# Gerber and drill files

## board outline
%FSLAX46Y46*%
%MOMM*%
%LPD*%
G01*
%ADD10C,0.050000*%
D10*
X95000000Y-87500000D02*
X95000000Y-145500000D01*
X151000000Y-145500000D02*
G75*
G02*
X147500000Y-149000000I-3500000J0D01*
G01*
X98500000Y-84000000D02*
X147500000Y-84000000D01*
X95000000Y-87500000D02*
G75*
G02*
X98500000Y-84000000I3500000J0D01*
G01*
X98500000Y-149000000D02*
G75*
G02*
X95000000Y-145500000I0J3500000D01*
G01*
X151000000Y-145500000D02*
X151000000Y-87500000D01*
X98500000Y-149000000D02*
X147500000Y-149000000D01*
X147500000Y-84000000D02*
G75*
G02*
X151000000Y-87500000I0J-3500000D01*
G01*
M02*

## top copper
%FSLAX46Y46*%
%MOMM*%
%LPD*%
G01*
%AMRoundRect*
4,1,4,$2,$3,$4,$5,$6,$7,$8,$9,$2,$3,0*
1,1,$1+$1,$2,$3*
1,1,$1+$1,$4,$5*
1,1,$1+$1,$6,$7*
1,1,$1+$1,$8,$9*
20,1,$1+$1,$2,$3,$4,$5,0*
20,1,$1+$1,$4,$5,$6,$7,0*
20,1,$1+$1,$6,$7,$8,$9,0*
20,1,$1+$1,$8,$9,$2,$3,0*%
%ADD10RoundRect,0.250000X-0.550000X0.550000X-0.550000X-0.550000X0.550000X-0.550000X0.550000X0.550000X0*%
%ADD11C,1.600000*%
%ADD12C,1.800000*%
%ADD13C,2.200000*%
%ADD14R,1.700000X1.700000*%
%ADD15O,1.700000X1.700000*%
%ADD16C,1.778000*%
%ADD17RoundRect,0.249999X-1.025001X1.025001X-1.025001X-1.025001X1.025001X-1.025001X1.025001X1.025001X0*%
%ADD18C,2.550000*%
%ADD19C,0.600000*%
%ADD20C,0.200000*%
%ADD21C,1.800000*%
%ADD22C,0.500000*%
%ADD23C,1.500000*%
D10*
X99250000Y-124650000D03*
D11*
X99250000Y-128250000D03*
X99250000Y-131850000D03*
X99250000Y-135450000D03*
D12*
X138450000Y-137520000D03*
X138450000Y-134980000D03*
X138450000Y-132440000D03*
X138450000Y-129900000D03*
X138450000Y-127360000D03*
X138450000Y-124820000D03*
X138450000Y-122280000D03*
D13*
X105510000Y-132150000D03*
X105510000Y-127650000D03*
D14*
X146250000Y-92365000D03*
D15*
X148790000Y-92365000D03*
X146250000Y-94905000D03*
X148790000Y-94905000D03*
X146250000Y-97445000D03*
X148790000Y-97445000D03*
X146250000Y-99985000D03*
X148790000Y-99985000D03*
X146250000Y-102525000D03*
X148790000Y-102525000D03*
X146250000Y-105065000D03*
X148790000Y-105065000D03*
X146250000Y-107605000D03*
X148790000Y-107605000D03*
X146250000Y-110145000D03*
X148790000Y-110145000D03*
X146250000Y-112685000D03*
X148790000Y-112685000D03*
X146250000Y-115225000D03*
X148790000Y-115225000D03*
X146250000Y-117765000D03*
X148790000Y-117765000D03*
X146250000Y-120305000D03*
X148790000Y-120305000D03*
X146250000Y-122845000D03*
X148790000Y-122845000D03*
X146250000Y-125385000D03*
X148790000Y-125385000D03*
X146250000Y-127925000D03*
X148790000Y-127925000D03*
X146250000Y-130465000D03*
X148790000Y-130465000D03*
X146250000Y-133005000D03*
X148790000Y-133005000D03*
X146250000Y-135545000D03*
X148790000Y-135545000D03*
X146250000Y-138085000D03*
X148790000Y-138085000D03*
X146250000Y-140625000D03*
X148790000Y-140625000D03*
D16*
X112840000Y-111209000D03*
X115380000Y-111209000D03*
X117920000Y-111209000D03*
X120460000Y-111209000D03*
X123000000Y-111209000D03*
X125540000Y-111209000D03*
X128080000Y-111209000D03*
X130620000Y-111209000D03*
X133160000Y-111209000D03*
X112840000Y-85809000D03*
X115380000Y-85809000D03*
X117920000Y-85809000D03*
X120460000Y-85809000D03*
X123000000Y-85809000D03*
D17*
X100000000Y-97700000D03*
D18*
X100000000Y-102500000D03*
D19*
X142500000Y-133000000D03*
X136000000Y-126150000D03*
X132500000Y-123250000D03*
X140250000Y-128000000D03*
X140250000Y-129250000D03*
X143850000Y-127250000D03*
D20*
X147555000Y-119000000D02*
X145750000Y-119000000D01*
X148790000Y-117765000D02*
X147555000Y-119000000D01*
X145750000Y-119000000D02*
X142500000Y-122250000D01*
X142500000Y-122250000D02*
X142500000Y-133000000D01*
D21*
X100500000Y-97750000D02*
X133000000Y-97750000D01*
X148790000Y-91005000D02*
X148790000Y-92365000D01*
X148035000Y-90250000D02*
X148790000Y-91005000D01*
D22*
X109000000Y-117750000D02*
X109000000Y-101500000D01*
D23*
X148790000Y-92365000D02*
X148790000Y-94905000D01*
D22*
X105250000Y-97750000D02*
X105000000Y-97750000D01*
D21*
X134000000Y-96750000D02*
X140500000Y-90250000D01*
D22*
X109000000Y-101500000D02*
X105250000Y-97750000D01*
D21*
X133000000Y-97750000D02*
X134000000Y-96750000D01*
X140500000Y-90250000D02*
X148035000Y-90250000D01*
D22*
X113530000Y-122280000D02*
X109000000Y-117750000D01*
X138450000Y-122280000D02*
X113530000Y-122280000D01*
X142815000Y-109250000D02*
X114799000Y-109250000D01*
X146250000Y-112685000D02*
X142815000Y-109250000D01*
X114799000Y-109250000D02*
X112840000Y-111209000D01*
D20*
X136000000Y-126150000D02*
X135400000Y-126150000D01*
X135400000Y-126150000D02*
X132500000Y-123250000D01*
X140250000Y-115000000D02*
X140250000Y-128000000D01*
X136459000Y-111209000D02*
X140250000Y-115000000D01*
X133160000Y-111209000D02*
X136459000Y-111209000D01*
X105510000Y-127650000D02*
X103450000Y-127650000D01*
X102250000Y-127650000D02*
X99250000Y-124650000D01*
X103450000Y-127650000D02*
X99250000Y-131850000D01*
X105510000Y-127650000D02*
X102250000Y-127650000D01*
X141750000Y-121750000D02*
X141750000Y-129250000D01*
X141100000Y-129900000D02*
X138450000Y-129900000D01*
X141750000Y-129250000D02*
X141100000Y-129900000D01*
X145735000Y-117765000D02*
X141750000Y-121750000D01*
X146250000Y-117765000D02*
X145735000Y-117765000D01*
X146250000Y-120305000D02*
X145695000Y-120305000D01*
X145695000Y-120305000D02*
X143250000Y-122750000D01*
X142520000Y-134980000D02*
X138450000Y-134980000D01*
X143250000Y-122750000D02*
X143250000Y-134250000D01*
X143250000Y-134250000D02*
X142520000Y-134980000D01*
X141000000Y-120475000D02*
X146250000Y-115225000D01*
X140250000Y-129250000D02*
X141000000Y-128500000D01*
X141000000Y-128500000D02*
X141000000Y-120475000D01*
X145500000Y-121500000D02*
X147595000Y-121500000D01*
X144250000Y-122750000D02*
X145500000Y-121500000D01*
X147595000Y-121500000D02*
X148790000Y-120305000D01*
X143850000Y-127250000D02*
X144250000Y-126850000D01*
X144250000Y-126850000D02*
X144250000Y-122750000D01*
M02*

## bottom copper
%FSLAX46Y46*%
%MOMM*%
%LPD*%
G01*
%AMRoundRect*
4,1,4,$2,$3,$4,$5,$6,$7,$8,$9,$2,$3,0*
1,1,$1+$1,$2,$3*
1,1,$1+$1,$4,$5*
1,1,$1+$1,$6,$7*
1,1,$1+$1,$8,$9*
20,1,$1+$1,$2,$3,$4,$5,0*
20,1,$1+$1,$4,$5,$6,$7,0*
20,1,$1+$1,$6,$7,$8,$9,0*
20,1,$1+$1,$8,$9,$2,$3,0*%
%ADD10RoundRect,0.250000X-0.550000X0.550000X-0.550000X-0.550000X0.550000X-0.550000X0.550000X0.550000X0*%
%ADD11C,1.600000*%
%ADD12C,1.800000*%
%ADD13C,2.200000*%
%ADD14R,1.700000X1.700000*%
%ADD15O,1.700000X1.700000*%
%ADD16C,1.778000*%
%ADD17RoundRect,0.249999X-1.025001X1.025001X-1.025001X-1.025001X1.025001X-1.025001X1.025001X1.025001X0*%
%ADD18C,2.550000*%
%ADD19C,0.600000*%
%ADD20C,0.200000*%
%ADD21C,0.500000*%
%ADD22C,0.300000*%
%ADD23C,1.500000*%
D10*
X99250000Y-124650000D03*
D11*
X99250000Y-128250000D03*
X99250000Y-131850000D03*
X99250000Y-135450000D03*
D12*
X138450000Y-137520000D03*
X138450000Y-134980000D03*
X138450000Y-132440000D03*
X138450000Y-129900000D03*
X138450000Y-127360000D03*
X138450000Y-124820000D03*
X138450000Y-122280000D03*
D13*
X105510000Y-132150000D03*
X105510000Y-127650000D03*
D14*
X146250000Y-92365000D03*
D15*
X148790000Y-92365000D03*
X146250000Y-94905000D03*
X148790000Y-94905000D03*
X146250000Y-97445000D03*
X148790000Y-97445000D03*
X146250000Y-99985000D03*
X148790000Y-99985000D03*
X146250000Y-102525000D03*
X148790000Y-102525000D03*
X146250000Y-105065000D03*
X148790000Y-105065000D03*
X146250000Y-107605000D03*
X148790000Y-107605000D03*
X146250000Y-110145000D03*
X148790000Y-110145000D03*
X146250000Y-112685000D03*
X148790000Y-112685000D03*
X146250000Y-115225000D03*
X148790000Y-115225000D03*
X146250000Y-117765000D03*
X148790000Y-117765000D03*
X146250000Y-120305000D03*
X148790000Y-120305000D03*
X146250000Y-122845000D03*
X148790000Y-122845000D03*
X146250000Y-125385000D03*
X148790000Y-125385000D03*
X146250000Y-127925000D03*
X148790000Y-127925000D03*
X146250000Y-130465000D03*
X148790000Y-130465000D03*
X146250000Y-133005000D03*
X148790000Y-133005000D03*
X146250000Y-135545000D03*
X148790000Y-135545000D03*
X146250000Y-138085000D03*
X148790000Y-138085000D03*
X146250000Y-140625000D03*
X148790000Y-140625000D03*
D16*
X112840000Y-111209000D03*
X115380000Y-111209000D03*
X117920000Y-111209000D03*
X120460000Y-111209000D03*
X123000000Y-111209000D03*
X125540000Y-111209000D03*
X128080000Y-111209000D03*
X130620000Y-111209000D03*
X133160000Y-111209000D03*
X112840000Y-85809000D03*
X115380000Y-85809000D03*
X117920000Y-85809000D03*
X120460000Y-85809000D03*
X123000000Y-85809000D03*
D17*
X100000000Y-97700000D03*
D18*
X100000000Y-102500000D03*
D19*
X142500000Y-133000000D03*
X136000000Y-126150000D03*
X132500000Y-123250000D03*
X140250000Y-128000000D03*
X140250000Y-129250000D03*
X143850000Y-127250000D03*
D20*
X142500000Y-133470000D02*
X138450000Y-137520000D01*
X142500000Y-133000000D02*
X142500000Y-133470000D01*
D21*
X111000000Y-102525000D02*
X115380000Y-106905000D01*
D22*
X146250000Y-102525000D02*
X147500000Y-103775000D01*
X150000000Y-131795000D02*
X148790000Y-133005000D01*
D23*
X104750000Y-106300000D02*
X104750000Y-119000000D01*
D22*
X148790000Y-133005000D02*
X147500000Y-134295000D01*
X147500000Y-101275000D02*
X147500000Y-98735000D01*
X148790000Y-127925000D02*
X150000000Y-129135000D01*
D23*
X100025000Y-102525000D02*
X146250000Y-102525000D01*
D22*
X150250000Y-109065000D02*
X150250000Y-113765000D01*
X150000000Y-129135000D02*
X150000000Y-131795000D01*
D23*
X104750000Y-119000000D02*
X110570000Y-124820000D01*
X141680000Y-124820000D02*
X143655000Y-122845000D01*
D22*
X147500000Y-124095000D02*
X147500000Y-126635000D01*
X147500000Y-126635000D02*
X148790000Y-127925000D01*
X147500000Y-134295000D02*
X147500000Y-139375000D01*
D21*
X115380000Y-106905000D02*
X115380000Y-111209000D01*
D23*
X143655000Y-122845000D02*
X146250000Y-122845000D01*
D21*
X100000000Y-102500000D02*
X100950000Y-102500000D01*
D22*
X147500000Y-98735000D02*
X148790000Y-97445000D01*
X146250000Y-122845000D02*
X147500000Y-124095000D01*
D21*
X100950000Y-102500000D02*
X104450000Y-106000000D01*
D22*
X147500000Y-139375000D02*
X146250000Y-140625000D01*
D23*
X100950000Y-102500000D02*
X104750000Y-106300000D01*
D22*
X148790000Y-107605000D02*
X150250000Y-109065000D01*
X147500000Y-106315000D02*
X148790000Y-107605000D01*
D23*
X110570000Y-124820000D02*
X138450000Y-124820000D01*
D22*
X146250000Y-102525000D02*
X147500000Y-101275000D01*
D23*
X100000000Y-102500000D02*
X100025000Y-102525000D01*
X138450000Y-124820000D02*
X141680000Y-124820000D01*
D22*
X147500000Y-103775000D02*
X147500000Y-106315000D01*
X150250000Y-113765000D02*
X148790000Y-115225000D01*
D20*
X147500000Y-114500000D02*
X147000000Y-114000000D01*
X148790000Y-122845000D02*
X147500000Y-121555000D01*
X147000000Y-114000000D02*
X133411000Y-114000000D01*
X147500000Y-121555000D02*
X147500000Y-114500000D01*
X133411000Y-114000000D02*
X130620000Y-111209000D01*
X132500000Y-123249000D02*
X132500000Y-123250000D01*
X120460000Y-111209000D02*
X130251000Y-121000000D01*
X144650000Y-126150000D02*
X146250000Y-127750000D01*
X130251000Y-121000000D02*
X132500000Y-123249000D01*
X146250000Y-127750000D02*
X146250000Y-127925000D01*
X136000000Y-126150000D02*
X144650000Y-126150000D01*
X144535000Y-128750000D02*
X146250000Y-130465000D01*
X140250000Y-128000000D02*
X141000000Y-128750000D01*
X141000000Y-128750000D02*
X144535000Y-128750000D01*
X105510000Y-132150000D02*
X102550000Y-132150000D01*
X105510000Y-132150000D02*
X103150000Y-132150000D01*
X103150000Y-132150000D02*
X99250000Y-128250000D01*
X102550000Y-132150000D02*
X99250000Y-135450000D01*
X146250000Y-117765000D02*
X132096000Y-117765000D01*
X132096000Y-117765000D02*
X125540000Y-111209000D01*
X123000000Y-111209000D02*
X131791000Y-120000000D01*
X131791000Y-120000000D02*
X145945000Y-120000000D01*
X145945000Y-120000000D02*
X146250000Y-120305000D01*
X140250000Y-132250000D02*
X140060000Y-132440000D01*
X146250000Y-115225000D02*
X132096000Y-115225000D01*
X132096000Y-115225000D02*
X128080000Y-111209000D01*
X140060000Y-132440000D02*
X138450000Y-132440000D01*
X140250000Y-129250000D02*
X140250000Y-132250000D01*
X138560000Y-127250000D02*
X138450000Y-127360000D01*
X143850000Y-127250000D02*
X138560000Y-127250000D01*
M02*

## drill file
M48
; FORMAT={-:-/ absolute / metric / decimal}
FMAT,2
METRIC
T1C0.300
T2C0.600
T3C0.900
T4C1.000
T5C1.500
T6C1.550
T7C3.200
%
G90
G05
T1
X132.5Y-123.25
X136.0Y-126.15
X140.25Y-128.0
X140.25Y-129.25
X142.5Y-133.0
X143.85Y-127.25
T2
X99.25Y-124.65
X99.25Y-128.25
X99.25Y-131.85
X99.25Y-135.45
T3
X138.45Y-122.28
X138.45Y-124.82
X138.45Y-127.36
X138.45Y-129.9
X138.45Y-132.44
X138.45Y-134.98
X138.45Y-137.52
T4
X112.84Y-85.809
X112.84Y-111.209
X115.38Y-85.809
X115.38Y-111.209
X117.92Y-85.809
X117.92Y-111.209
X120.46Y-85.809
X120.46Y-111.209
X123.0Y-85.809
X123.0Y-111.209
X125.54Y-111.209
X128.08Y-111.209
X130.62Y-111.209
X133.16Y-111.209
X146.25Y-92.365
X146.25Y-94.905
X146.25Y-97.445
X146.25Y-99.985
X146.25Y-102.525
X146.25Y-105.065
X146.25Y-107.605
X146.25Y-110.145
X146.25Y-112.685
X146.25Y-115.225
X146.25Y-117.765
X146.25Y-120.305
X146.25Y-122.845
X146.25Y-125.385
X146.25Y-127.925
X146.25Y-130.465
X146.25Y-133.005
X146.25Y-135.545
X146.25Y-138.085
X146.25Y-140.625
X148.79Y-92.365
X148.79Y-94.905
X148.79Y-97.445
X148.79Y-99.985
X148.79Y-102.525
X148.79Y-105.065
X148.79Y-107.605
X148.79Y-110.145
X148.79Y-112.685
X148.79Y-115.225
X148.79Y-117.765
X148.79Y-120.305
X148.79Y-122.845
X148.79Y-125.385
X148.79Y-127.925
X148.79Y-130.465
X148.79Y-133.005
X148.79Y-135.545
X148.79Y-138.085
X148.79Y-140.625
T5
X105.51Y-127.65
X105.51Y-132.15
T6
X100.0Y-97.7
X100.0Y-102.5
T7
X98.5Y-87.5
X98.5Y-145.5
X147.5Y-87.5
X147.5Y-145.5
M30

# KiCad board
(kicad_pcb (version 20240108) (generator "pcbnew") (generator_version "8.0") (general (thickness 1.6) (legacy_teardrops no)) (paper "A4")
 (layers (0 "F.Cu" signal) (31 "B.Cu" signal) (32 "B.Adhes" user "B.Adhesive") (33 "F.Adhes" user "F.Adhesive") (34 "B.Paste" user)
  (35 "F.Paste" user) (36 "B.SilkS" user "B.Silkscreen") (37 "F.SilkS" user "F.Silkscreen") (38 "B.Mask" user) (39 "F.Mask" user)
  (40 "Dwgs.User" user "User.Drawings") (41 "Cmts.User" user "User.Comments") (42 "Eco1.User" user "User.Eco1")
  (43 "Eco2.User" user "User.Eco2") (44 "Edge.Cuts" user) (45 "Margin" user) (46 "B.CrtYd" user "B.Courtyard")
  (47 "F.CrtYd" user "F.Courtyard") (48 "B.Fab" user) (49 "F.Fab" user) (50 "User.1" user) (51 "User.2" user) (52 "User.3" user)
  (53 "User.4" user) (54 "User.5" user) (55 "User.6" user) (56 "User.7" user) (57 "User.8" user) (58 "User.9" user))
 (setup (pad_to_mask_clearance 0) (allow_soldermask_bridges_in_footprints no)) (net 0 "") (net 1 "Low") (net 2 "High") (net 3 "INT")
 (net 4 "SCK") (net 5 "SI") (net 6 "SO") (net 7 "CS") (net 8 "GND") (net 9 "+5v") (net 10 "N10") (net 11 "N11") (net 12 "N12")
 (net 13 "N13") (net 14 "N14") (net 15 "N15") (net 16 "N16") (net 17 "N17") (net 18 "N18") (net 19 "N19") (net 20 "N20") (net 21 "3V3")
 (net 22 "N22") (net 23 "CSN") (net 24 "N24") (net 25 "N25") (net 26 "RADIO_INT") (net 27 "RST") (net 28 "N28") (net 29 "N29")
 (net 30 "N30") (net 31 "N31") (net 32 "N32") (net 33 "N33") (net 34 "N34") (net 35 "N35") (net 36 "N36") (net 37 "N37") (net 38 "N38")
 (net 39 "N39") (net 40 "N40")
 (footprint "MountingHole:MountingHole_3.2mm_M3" (layer "F.Cu") (at 147.5 87.5 180)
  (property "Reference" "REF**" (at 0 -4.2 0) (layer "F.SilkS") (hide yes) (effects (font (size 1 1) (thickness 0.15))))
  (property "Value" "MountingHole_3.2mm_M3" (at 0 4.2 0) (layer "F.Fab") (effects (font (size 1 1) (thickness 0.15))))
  (pad "" np_thru_hole circle (at 0 0 180) (size 3.2 3.2) (drill 3.2) (layers "*.Cu" "*.Mask")))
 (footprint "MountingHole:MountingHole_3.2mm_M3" (layer "F.Cu") (at 98.5 145.5 180)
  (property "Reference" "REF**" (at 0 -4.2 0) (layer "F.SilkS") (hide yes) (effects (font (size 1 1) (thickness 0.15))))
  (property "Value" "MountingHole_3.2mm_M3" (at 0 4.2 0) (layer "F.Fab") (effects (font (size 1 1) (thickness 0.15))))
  (pad "" np_thru_hole circle (at 0 0 180) (size 3.2 3.2) (drill 3.2) (layers "*.Cu" "*.Mask")))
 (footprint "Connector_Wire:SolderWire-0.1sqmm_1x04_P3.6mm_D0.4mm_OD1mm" (layer "F.Cu") (at 99.25 124.65 -90)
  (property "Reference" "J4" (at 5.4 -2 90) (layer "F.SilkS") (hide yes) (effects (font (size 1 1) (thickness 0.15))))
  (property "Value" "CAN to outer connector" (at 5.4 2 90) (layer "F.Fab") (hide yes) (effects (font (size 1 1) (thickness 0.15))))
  (pad "1" thru_hole roundrect (at 0 0 270) (size 1.6 1.6) (drill 0.6) (layers "*.Cu" "*.Mask") (remove_unused_layers no)
   (roundrect_rratio 0.15625) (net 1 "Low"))
  (pad "2" thru_hole circle (at 3.6 0 270) (size 1.6 1.6) (drill 0.6) (layers "*.Cu" "*.Mask") (remove_unused_layers no) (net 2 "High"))
  (pad "3" thru_hole circle (at 7.2 0 270) (size 1.6 1.6) (drill 0.6) (layers "*.Cu" "*.Mask") (remove_unused_layers no) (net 1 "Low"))
  (pad "4" thru_hole circle (at 10.8 0 270) (size 1.6 1.6) (drill 0.6) (layers "*.Cu" "*.Mask") (remove_unused_layers no) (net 2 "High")))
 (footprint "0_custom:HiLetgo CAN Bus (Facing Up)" (layer "F.Cu") (at 128.5 127.5 180)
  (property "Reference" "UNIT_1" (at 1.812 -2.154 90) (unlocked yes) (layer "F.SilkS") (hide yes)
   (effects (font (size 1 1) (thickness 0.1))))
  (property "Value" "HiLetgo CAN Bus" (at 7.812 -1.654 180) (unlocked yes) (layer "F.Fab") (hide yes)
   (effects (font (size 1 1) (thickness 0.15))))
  (pad "1" thru_hole circle (at -9.95 -10.02) (size 1.8 1.8) (drill 0.9) (layers "*.Cu" "*.Mask") (remove_unused_layers no) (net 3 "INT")
   (solder_mask_margin 0.102))
  (pad "2" thru_hole circle (at -9.95 -7.48) (size 1.8 1.8) (drill 0.9) (layers "*.Cu" "*.Mask") (remove_unused_layers no) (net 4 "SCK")
   (solder_mask_margin 0.102))
  (pad "3" thru_hole circle (at -9.95 -4.94) (size 1.8 1.8) (drill 0.9) (layers "*.Cu" "*.Mask") (remove_unused_layers no) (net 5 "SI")
   (solder_mask_margin 0.102))
  (pad "4" thru_hole circle (at -9.95 -2.4) (size 1.8 1.8) (drill 0.9) (layers "*.Cu" "*.Mask") (remove_unused_layers no) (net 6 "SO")
   (solder_mask_margin 0.102))
  (pad "5" thru_hole circle (at -9.95 0.14) (size 1.8 1.8) (drill 0.9) (layers "*.Cu" "*.Mask") (remove_unused_layers no) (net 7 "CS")
   (solder_mask_margin 0.102))
  (pad "6" thru_hole circle (at -9.95 2.68) (size 1.8 1.8) (drill 0.9) (layers "*.Cu" "*.Mask") (remove_unused_layers no) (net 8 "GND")
   (solder_mask_margin 0.102))
  (pad "7" thru_hole circle (at -9.95 5.22) (size 1.8 1.8) (drill 0.9) (layers "*.Cu" "*.Mask") (remove_unused_layers no) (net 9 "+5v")
   (solder_mask_margin 0.102))
  (pad "8" thru_hole circle (at 22.99 -4.65) (size 2.2 2.2) (drill 1.5) (layers "*.Cu" "*.Mask") (remove_unused_layers no) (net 2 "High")
   (solder_mask_margin 0.102))
  (pad "9" thru_hole circle (at 22.99 -0.15) (size 2.2 2.2) (drill 1.5) (layers "*.Cu" "*.Mask") (remove_unused_layers no) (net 1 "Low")
   (solder_mask_margin 0.102)))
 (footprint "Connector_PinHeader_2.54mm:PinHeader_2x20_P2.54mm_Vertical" (layer "F.Cu") (at 146.25 92.365)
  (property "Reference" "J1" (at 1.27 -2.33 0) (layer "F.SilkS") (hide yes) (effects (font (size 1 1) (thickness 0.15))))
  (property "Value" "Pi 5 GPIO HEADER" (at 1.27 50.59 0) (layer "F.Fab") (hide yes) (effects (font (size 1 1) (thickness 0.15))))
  (pad "1" thru_hole rect (at 0 0) (size 1.7 1.7) (drill 1) (layers "*.Cu" "*.Mask") (remove_unused_layers no) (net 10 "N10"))
  (pad "2" thru_hole oval (at 2.54 0) (size 1.7 1.7) (drill 1) (layers "*.Cu" "*.Mask") (remove_unused_layers no) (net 9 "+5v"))
  (pad "3" thru_hole oval (at 0 2.54) (size 1.7 1.7) (drill 1) (layers "*.Cu" "*.Mask") (remove_unused_layers no) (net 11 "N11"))
  (pad "4" thru_hole oval (at 2.54 2.54) (size 1.7 1.7) (drill 1) (layers "*.Cu" "*.Mask") (remove_unused_layers no) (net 9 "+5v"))
  (pad "5" thru_hole oval (at 0 5.08) (size 1.7 1.7) (drill 1) (layers "*.Cu" "*.Mask") (remove_unused_layers no) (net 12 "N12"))
  (pad "6" thru_hole oval (at 2.54 5.08) (size 1.7 1.7) (drill 1) (layers "*.Cu" "*.Mask") (remove_unused_layers no) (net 8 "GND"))
  (pad "7" thru_hole oval (at 0 7.62) (size 1.7 1.7) (drill 1) (layers "*.Cu" "*.Mask") (remove_unused_layers no) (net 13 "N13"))
  (pad "8" thru_hole oval (at 2.54 7.62) (size 1.7 1.7) (drill 1) (layers "*.Cu" "*.Mask") (remove_unused_layers no) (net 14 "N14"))
  (pad "9" thru_hole oval (at 0 10.16) (size 1.7 1.7) (drill 1) (layers "*.Cu" "*.Mask") (remove_unused_layers no) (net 8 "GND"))
  (pad "10" thru_hole oval (at 2.54 10.16) (size 1.7 1.7) (drill 1) (layers "*.Cu" "*.Mask") (remove_unused_layers no) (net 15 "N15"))
  (pad "11" thru_hole oval (at 0 12.7) (size 1.7 1.7) (drill 1) (layers "*.Cu" "*.Mask") (remove_unused_layers no) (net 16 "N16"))
  (pad "12" thru_hole oval (at 2.54 12.7) (size 1.7 1.7) (drill 1) (layers "*.Cu" "*.Mask") (remove_unused_layers no) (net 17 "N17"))
  (pad "13" thru_hole oval (at 0 15.24) (size 1.7 1.7) (drill 1) (layers "*.Cu" "*.Mask") (remove_unused_layers no) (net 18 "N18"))
  (pad "14" thru_hole oval (at 2.54 15.24) (size 1.7 1.7) (drill 1) (layers "*.Cu" "*.Mask") (remove_unused_layers no) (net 8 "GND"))
  (pad "15" thru_hole oval (at 0 17.78) (size 1.7 1.7) (drill 1) (layers "*.Cu" "*.Mask") (remove_unused_layers no) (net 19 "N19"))
  (pad "16" thru_hole oval (at 2.54 17.78) (size 1.7 1.7) (drill 1) (layers "*.Cu" "*.Mask") (remove_unused_layers no) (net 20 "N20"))
  (pad "17" thru_hole oval (at 0 20.32) (size 1.7 1.7) (drill 1) (layers "*.Cu" "*.Mask") (remove_unused_layers no) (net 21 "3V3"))
  (pad "18" thru_hole oval (at 2.54 20.32) (size 1.7 1.7) (drill 1) (layers "*.Cu" "*.Mask") (remove_unused_layers no) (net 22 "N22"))
  (pad "19" thru_hole oval (at 0 22.86) (size 1.7 1.7) (drill 1) (layers "*.Cu" "*.Mask") (remove_unused_layers no) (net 5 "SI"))
  (pad "20" thru_hole oval (at 2.54 22.86) (size 1.7 1.7) (drill 1) (layers "*.Cu" "*.Mask") (remove_unused_layers no) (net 8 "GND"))
  (pad "21" thru_hole oval (at 0 25.4) (size 1.7 1.7) (drill 1) (layers "*.Cu" "*.Mask") (remove_unused_layers no) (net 6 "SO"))
  (pad "22" thru_hole oval (at 2.54 25.4) (size 1.7 1.7) (drill 1) (layers "*.Cu" "*.Mask") (remove_unused_layers no) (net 3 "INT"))
  (pad "23" thru_hole oval (at 0 27.94) (size 1.7 1.7) (drill 1) (layers "*.Cu" "*.Mask") (remove_unused_layers no) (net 4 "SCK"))
  (pad "24" thru_hole oval (at 2.54 27.94) (size 1.7 1.7) (drill 1) (layers "*.Cu" "*.Mask") (remove_unused_layers no) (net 7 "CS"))
  (pad "25" thru_hole oval (at 0 30.48) (size 1.7 1.7) (drill 1) (layers "*.Cu" "*.Mask") (remove_unused_layers no) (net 8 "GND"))
  (pad "26" thru_hole oval (at 2.54 30.48) (size 1.7 1.7) (drill 1) (layers "*.Cu" "*.Mask") (remove_unused_layers no) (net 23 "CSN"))
  (pad "27" thru_hole oval (at 0 33.02) (size 1.7 1.7) (drill 1) (layers "*.Cu" "*.Mask") (remove_unused_layers no) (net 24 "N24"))
  (pad "28" thru_hole oval (at 2.54 33.02) (size 1.7 1.7) (drill 1) (layers "*.Cu" "*.Mask") (remove_unused_layers no) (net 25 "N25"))
  (pad "29" thru_hole oval (at 0 35.56) (size 1.7 1.7) (drill 1) (layers "*.Cu" "*.Mask") (remove_unused_layers no) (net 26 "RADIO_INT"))
  (pad "30" thru_hole oval (at 2.54 35.56) (size 1.7 1.7) (drill 1) (layers "*.Cu" "*.Mask") (remove_unused_layers no) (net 8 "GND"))
  (pad "31" thru_hole oval (at 0 38.1) (size 1.7 1.7) (drill 1) (layers "*.Cu" "*.Mask") (remove_unused_layers no) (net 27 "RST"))
  (pad "32" thru_hole oval (at 2.54 38.1) (size 1.7 1.7) (drill 1) (layers "*.Cu" "*.Mask") (remove_unused_layers no) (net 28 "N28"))
  (pad "33" thru_hole oval (at 0 40.64) (size 1.7 1.7) (drill 1) (layers "*.Cu" "*.Mask") (remove_unused_layers no) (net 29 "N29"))
  (pad "34" thru_hole oval (at 2.54 40.64) (size 1.7 1.7) (drill 1) (layers "*.Cu" "*.Mask") (remove_unused_layers no) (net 8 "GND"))
  (pad "35" thru_hole oval (at 0 43.18) (size 1.7 1.7) (drill 1) (layers "*.Cu" "*.Mask") (remove_unused_layers no) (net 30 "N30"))
  (pad "36" thru_hole oval (at 2.54 43.18) (size 1.7 1.7) (drill 1) (layers "*.Cu" "*.Mask") (remove_unused_layers no) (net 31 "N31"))
  (pad "37" thru_hole oval (at 0 45.72) (size 1.7 1.7) (drill 1) (layers "*.Cu" "*.Mask") (remove_unused_layers no) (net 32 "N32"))
  (pad "38" thru_hole oval (at 2.54 45.72) (size 1.7 1.7) (drill 1) (layers "*.Cu" "*.Mask") (remove_unused_layers no) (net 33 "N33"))
  (pad "39" thru_hole oval (at 0 48.26) (size 1.7 1.7) (drill 1) (layers "*.Cu" "*.Mask") (remove_unused_layers no) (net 8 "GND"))
  (pad "40" thru_hole oval (at 2.54 48.26) (size 1.7 1.7) (drill 1) (layers "*.Cu" "*.Mask") (remove_unused_layers no) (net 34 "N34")))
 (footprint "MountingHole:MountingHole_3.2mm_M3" (layer "F.Cu") (at 98.5 87.5)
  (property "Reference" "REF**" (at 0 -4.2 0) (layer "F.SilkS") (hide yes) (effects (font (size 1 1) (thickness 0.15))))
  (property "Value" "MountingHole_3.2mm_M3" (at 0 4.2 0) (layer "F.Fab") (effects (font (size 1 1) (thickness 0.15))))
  (pad "" np_thru_hole circle (at 0 0) (size 3.2 3.2) (drill 3.2) (layers "*.Cu" "*.Mask")))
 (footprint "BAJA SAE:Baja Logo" (layer "F.Cu") (at 140 100.25 -90)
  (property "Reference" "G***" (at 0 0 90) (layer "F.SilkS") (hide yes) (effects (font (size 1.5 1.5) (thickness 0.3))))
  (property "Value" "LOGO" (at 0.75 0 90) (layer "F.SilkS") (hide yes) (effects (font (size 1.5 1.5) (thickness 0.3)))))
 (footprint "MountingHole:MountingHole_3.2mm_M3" (layer "F.Cu") (at 147.5 145.5)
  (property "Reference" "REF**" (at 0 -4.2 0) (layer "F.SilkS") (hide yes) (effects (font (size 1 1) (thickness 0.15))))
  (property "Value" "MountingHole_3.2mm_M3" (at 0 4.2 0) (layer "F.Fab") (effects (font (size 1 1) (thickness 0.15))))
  (pad "" np_thru_hole circle (at 0 0) (size 3.2 3.2) (drill 3.2) (layers "*.Cu" "*.Mask")))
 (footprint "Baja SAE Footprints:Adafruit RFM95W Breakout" (layer "F.Cu") (at 123 79.205)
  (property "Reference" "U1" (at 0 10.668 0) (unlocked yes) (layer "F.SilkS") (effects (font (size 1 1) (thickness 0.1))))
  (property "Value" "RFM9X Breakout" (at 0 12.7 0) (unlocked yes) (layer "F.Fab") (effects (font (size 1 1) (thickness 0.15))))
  (pad "1" thru_hole circle (at -10.16 32.004) (size 1.778 1.778) (drill 1) (layers "*.Cu" "*.Mask") (remove_unused_layers no)
   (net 21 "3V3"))
  (pad "2" thru_hole circle (at -7.62 32.004) (size 1.778 1.778) (drill 1) (layers "*.Cu" "*.Mask") (remove_unused_layers no) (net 8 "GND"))
  (pad "3" thru_hole circle (at -5.08 32.004) (size 1.778 1.778) (drill 1) (layers "*.Cu" "*.Mask") (remove_unused_layers no) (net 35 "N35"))
  (pad "4" thru_hole circle (at -2.54 32.004) (size 1.778 1.778) (drill 1) (layers "*.Cu" "*.Mask") (remove_unused_layers no)
   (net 26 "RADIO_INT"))
  (pad "5" thru_hole circle (at 0 32.004) (size 1.778 1.778) (drill 1) (layers "*.Cu" "*.Mask") (remove_unused_layers no) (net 4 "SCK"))
  (pad "6" thru_hole circle (at 2.54 32.004) (size 1.778 1.778) (drill 1) (layers "*.Cu" "*.Mask") (remove_unused_layers no) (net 6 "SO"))
  (pad "7" thru_hole circle (at 5.08 32.004) (size 1.778 1.778) (drill 1) (layers "*.Cu" "*.Mask") (remove_unused_layers no) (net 5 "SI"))
  (pad "8" thru_hole circle (at 7.62 32.004) (size 1.778 1.778) (drill 1) (layers "*.Cu" "*.Mask") (remove_unused_layers no) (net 23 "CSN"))
  (pad "9" thru_hole circle (at 10.16 32.004) (size 1.778 1.778) (drill 1) (layers "*.Cu" "*.Mask") (remove_unused_layers no) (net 27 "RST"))
  (pad "10" thru_hole circle (at -10.16 6.604) (size 1.778 1.778) (drill 1) (layers "*.Cu" "*.Mask") (remove_unused_layers no)
   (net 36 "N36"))
  (pad "11" thru_hole circle (at -7.62 6.604) (size 1.778 1.778) (drill 1) (layers "*.Cu" "*.Mask") (remove_unused_layers no) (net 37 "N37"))
  (pad "12" thru_hole circle (at -5.08 6.604) (size 1.778 1.778) (drill 1) (layers "*.Cu" "*.Mask") (remove_unused_layers no) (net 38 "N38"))
  (pad "13" thru_hole circle (at -2.54 6.604) (size 1.778 1.778) (drill 1) (layers "*.Cu" "*.Mask") (remove_unused_layers no) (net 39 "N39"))
  (pad "14" thru_hole circle (at 0 6.604) (size 1.778 1.778) (drill 1) (layers "*.Cu" "*.Mask") (remove_unused_layers no) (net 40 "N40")))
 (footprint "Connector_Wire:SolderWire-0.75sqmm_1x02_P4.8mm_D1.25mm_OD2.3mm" (layer "F.Cu") (at 100 97.7 -90)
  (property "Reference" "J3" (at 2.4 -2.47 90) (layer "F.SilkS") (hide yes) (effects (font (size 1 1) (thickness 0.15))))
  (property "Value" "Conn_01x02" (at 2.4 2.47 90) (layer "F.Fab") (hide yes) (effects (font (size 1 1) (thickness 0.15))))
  (pad "1" thru_hole roundrect (at 0 0 270) (size 2.55 2.55) (drill 1.55) (layers "*.Cu" "*.Mask") (remove_unused_layers no)
   (roundrect_rratio 0.098039) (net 9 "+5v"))
  (pad "2" thru_hole circle (at 4.8 0 270) (size 2.55 2.55) (drill 1.55) (layers "*.Cu" "*.Mask") (remove_unused_layers no) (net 8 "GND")))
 (gr_line (start 95 87.5) (end 95 145.5) (stroke (width 0.05) (type default)) (layer "Edge.Cuts"))
 (gr_arc (start 151 145.5) (mid 149.974874 147.974874) (end 147.5 149) (stroke (width 0.05) (type default)) (layer "Edge.Cuts"))
 (gr_line (start 98.5 84) (end 147.5 84) (stroke (width 0.05) (type default)) (layer "Edge.Cuts"))
 (gr_arc (start 95 87.5) (mid 96.025126 85.025126) (end 98.5 84) (stroke (width 0.05) (type default)) (layer "Edge.Cuts"))
 (gr_arc (start 98.5 149) (mid 96.025126 147.974874) (end 95 145.5) (stroke (width 0.05) (type default)) (layer "Edge.Cuts"))
 (gr_line (start 151 145.5) (end 151 87.5) (stroke (width 0.05) (type default)) (layer "Edge.Cuts"))
 (gr_line (start 98.5 149) (end 147.5 149) (stroke (width 0.05) (type default)) (layer "Edge.Cuts"))
 (gr_arc (start 147.5 84) (mid 149.974874 85.025126) (end 151 87.5) (stroke (width 0.05) (type default)) (layer "Edge.Cuts"))
 (segment (start 147.555 119) (end 145.75 119) (width 0.2) (layer "F.Cu") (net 3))
 (segment (start 148.79 117.765) (end 147.555 119) (width 0.2) (layer "F.Cu") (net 3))
 (segment (start 145.75 119) (end 142.5 122.25) (width 0.2) (layer "F.Cu") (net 3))
 (segment (start 142.5 122.25) (end 142.5 133) (width 0.2) (layer "F.Cu") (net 3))
 (via (at 142.5 133) (size 0.6) (drill 0.3) (layers "F.Cu" "B.Cu") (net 3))
 (segment (start 142.5 133.47) (end 138.45 137.52) (width 0.2) (layer "B.Cu") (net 3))
 (segment (start 142.5 133) (end 142.5 133.47) (width 0.2) (layer "B.Cu") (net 3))
 (segment (start 100.5 97.75) (end 133 97.75) (width 1.8) (layer "F.Cu") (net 9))
 (segment (start 148.79 91.005) (end 148.79 92.365) (width 1.8) (layer "F.Cu") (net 9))
 (segment (start 148.035 90.25) (end 148.79 91.005) (width 1.8) (layer "F.Cu") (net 9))
 (segment (start 109 117.75) (end 109 101.5) (width 0.5) (layer "F.Cu") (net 9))
 (segment (start 148.79 92.365) (end 148.79 94.905) (width 1.5) (layer "F.Cu") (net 9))
 (segment (start 105.25 97.75) (end 105 97.75) (width 0.5) (layer "F.Cu") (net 9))
 (segment (start 134 96.75) (end 140.5 90.25) (width 1.8) (layer "F.Cu") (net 9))
 (segment (start 109 101.5) (end 105.25 97.75) (width 0.5) (layer "F.Cu") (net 9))
 (segment (start 133 97.75) (end 134 96.75) (width 1.8) (layer "F.Cu") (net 9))
 (segment (start 140.5 90.25) (end 148.035 90.25) (width 1.8) (layer "F.Cu") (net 9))
 (segment (start 113.53 122.28) (end 109 117.75) (width 0.5) (layer "F.Cu") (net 9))
 (segment (start 138.45 122.28) (end 113.53 122.28) (width 0.5) (layer "F.Cu") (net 9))
 (segment (start 111 102.525) (end 115.38 106.905) (width 0.5) (layer "B.Cu") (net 8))
 (segment (start 146.25 102.525) (end 147.5 103.775) (width 0.3) (layer "B.Cu") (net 8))
 (segment (start 150 131.795) (end 148.79 133.005) (width 0.3) (layer "B.Cu") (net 8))
 (segment (start 104.75 106.3) (end 104.75 119) (width 1.5) (layer "B.Cu") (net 8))
 (segment (start 148.79 133.005) (end 147.5 134.295) (width 0.3) (layer "B.Cu") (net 8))
 (segment (start 147.5 101.275) (end 147.5 98.735) (width 0.3) (layer "B.Cu") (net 8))
 (segment (start 148.79 127.925) (end 150 129.135) (width 0.3) (layer "B.Cu") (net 8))
 (segment (start 100.025 102.525) (end 146.25 102.525) (width 1.5) (layer "B.Cu") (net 8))
 (segment (start 150.25 109.065) (end 150.25 113.765) (width 0.3) (layer "B.Cu") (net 8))
 (segment (start 150 129.135) (end 150 131.795) (width 0.3) (layer "B.Cu") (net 8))
 (segment (start 104.75 119) (end 110.57 124.82) (width 1.5) (layer "B.Cu") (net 8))
 (segment (start 141.68 124.82) (end 143.655 122.845) (width 1.5) (layer "B.Cu") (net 8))
 (segment (start 147.5 124.095) (end 147.5 126.635) (width 0.3) (layer "B.Cu") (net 8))
 (segment (start 147.5 126.635) (end 148.79 127.925) (width 0.3) (layer "B.Cu") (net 8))
 (segment (start 147.5 134.295) (end 147.5 139.375) (width 0.3) (layer "B.Cu") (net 8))
 (segment (start 115.38 106.905) (end 115.38 111.209) (width 0.5) (layer "B.Cu") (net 8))
 (segment (start 143.655 122.845) (end 146.25 122.845) (width 1.5) (layer "B.Cu") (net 8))
 (segment (start 100 102.5) (end 100.95 102.5) (width 0.5) (layer "B.Cu") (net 8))
 (segment (start 147.5 98.735) (end 148.79 97.445) (width 0.3) (layer "B.Cu") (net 8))
 (segment (start 146.25 122.845) (end 147.5 124.095) (width 0.3) (layer "B.Cu") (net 8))
 (segment (start 100.95 102.5) (end 104.45 106) (width 0.5) (layer "B.Cu") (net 8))
 (segment (start 147.5 139.375) (end 146.25 140.625) (width 0.3) (layer "B.Cu") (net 8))
 (segment (start 100.95 102.5) (end 104.75 106.3) (width 1.5) (layer "B.Cu") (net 8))
 (segment (start 148.79 107.605) (end 150.25 109.065) (width 0.3) (layer "B.Cu") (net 8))
 (segment (start 147.5 106.315) (end 148.79 107.605) (width 0.3) (layer "B.Cu") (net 8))
 (segment (start 110.57 124.82) (end 138.45 124.82) (width 1.5) (layer "B.Cu") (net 8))
 (segment (start 146.25 102.525) (end 147.5 101.275) (width 0.3) (layer "B.Cu") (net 8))
 (segment (start 100 102.5) (end 100.025 102.525) (width 1.5) (layer "B.Cu") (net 8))
 (segment (start 138.45 124.82) (end 141.68 124.82) (width 1.5) (layer "B.Cu") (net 8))
 (segment (start 147.5 103.775) (end 147.5 106.315) (width 0.3) (layer "B.Cu") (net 8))
 (segment (start 150.25 113.765) (end 148.79 115.225) (width 0.3) (layer "B.Cu") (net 8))
 (segment (start 147.5 114.5) (end 147 114) (width 0.2) (layer "B.Cu") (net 23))
 (segment (start 148.79 122.845) (end 147.5 121.555) (width 0.2) (layer "B.Cu") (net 23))
 (segment (start 147 114) (end 133.411 114) (width 0.2) (layer "B.Cu") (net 23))
 (segment (start 147.5 121.555) (end 147.5 114.5) (width 0.2) (layer "B.Cu") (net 23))
 (segment (start 133.411 114) (end 130.62 111.209) (width 0.2) (layer "B.Cu") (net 23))
 (segment (start 142.815 109.25) (end 114.799 109.25) (width 0.5) (layer "F.Cu") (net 21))
 (segment (start 146.25 112.685) (end 142.815 109.25) (width 0.5) (layer "F.Cu") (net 21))
 (segment (start 114.799 109.25) (end 112.84 111.209) (width 0.5) (layer "F.Cu") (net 21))
 (segment (start 136 126.15) (end 135.4 126.15) (width 0.2) (layer "F.Cu") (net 26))
 (segment (start 135.4 126.15) (end 132.5 123.25) (width 0.2) (layer "F.Cu") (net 26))
 (via (at 136 126.15) (size 0.6) (drill 0.3) (layers "F.Cu" "B.Cu") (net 26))
 (via (at 132.5 123.25) (size 0.6) (drill 0.3) (layers "F.Cu" "B.Cu") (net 26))
 (segment (start 132.5 123.249) (end 132.5 123.25) (width 0.2) (layer "B.Cu") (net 26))
 (segment (start 120.46 111.209) (end 130.251 121) (width 0.2) (layer "B.Cu") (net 26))
 (segment (start 144.65 126.15) (end 146.25 127.75) (width 0.2) (layer "B.Cu") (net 26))
 (segment (start 130.251 121) (end 132.5 123.249) (width 0.2) (layer "B.Cu") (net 26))
 (segment (start 146.25 127.75) (end 146.25 127.925) (width 0.2) (layer "B.Cu") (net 26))
 (segment (start 136 126.15) (end 144.65 126.15) (width 0.2) (layer "B.Cu") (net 26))
 (segment (start 140.25 115) (end 140.25 128) (width 0.2) (layer "F.Cu") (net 27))
 (segment (start 136.459 111.209) (end 140.25 115) (width 0.2) (layer "F.Cu") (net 27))
 (segment (start 133.16 111.209) (end 136.459 111.209) (width 0.2) (layer "F.Cu") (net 27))
 (via (at 140.25 128) (size 0.6) (drill 0.3) (layers "F.Cu" "B.Cu") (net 27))
 (segment (start 144.535 128.75) (end 146.25 130.465) (width 0.2) (layer "B.Cu") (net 27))
 (segment (start 140.25 128) (end 141 128.75) (width 0.2) (layer "B.Cu") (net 27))
 (segment (start 141 128.75) (end 144.535 128.75) (width 0.2) (layer "B.Cu") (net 27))
 (segment (start 105.51 132.15) (end 102.55 132.15) (width 0.2) (layer "B.Cu") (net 2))
 (segment (start 105.51 132.15) (end 103.15 132.15) (width 0.2) (layer "B.Cu") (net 2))
 (segment (start 103.15 132.15) (end 99.25 128.25) (width 0.2) (layer "B.Cu") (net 2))
 (segment (start 102.55 132.15) (end 99.25 135.45) (width 0.2) (layer "B.Cu") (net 2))
 (segment (start 105.51 127.65) (end 103.45 127.65) (width 0.2) (layer "F.Cu") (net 1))
 (segment (start 102.25 127.65) (end 99.25 124.65) (width 0.2) (layer "F.Cu") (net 1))
 (segment (start 103.45 127.65) (end 99.25 131.85) (width 0.2) (layer "F.Cu") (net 1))
 (segment (start 105.51 127.65) (end 102.25 127.65) (width 0.2) (layer "F.Cu") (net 1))
 (segment (start 141.75 121.75) (end 141.75 129.25) (width 0.2) (layer "F.Cu") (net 6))
 (segment (start 141.1 129.9) (end 138.45 129.9) (width 0.2) (layer "F.Cu") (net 6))
 (segment (start 141.75 129.25) (end 141.1 129.9) (width 0.2) (layer "F.Cu") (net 6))
 (segment (start 145.735 117.765) (end 141.75 121.75) (width 0.2) (layer "F.Cu") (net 6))
 (segment (start 146.25 117.765) (end 145.735 117.765) (width 0.2) (layer "F.Cu") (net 6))
 (segment (start 146.25 117.765) (end 132.096 117.765) (width 0.2) (layer "B.Cu") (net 6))
 (segment (start 132.096 117.765) (end 125.54 111.209) (width 0.2) (layer "B.Cu") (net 6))
 (segment (start 146.25 120.305) (end 145.695 120.305) (width 0.2) (layer "F.Cu") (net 4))
 (segment (start 145.695 120.305) (end 143.25 122.75) (width 0.2) (layer "F.Cu") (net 4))
 (segment (start 142.52 134.98) (end 138.45 134.98) (width 0.2) (layer "F.Cu") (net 4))
 (segment (start 143.25 122.75) (end 143.25 134.25) (width 0.2) (layer "F.Cu") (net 4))
 (segment (start 143.25 134.25) (end 142.52 134.98) (width 0.2) (layer "F.Cu") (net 4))
 (segment (start 123 111.209) (end 131.791 120) (width 0.2) (layer "B.Cu") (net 4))
 (segment (start 131.791 120) (end 145.945 120) (width 0.2) (layer "B.Cu") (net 4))
 (segment (start 145.945 120) (end 146.25 120.305) (width 0.2) (layer "B.Cu") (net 4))
 (segment (start 141 120.475) (end 146.25 115.225) (width 0.2) (layer "F.Cu") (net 5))
 (segment (start 140.25 129.25) (end 141 128.5) (width 0.2) (layer "F.Cu") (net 5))
 (segment (start 141 128.5) (end 141 120.475) (width 0.2) (layer "F.Cu") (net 5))
 (via (at 140.25 129.25) (size 0.6) (drill 0.3) (layers "F.Cu" "B.Cu") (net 5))
 (segment (start 140.25 132.25) (end 140.06 132.44) (width 0.2) (layer "B.Cu") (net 5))
 (segment (start 146.25 115.225) (end 132.096 115.225) (width 0.2) (layer "B.Cu") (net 5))
 (segment (start 132.096 115.225) (end 128.08 111.209) (width 0.2) (layer "B.Cu") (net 5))
 (segment (start 140.06 132.44) (end 138.45 132.44) (width 0.2) (layer "B.Cu") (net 5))
 (segment (start 140.25 129.25) (end 140.25 132.25) (width 0.2) (layer "B.Cu") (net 5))
 (segment (start 145.5 121.5) (end 147.595 121.5) (width 0.2) (layer "F.Cu") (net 7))
 (segment (start 144.25 122.75) (end 145.5 121.5) (width 0.2) (layer "F.Cu") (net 7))
 (segment (start 147.595 121.5) (end 148.79 120.305) (width 0.2) (layer "F.Cu") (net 7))
 (segment (start 143.85 127.25) (end 144.25 126.85) (width 0.2) (layer "F.Cu") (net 7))
 (segment (start 144.25 126.85) (end 144.25 122.75) (width 0.2) (layer "F.Cu") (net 7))
 (via (at 143.85 127.25) (size 0.6) (drill 0.3) (layers "F.Cu" "B.Cu") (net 7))
 (segment (start 138.56 127.25) (end 138.45 127.36) (width 0.2) (layer "B.Cu") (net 7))
 (segment (start 143.85 127.25) (end 138.56 127.25) (width 0.2) (layer "B.Cu") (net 7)))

